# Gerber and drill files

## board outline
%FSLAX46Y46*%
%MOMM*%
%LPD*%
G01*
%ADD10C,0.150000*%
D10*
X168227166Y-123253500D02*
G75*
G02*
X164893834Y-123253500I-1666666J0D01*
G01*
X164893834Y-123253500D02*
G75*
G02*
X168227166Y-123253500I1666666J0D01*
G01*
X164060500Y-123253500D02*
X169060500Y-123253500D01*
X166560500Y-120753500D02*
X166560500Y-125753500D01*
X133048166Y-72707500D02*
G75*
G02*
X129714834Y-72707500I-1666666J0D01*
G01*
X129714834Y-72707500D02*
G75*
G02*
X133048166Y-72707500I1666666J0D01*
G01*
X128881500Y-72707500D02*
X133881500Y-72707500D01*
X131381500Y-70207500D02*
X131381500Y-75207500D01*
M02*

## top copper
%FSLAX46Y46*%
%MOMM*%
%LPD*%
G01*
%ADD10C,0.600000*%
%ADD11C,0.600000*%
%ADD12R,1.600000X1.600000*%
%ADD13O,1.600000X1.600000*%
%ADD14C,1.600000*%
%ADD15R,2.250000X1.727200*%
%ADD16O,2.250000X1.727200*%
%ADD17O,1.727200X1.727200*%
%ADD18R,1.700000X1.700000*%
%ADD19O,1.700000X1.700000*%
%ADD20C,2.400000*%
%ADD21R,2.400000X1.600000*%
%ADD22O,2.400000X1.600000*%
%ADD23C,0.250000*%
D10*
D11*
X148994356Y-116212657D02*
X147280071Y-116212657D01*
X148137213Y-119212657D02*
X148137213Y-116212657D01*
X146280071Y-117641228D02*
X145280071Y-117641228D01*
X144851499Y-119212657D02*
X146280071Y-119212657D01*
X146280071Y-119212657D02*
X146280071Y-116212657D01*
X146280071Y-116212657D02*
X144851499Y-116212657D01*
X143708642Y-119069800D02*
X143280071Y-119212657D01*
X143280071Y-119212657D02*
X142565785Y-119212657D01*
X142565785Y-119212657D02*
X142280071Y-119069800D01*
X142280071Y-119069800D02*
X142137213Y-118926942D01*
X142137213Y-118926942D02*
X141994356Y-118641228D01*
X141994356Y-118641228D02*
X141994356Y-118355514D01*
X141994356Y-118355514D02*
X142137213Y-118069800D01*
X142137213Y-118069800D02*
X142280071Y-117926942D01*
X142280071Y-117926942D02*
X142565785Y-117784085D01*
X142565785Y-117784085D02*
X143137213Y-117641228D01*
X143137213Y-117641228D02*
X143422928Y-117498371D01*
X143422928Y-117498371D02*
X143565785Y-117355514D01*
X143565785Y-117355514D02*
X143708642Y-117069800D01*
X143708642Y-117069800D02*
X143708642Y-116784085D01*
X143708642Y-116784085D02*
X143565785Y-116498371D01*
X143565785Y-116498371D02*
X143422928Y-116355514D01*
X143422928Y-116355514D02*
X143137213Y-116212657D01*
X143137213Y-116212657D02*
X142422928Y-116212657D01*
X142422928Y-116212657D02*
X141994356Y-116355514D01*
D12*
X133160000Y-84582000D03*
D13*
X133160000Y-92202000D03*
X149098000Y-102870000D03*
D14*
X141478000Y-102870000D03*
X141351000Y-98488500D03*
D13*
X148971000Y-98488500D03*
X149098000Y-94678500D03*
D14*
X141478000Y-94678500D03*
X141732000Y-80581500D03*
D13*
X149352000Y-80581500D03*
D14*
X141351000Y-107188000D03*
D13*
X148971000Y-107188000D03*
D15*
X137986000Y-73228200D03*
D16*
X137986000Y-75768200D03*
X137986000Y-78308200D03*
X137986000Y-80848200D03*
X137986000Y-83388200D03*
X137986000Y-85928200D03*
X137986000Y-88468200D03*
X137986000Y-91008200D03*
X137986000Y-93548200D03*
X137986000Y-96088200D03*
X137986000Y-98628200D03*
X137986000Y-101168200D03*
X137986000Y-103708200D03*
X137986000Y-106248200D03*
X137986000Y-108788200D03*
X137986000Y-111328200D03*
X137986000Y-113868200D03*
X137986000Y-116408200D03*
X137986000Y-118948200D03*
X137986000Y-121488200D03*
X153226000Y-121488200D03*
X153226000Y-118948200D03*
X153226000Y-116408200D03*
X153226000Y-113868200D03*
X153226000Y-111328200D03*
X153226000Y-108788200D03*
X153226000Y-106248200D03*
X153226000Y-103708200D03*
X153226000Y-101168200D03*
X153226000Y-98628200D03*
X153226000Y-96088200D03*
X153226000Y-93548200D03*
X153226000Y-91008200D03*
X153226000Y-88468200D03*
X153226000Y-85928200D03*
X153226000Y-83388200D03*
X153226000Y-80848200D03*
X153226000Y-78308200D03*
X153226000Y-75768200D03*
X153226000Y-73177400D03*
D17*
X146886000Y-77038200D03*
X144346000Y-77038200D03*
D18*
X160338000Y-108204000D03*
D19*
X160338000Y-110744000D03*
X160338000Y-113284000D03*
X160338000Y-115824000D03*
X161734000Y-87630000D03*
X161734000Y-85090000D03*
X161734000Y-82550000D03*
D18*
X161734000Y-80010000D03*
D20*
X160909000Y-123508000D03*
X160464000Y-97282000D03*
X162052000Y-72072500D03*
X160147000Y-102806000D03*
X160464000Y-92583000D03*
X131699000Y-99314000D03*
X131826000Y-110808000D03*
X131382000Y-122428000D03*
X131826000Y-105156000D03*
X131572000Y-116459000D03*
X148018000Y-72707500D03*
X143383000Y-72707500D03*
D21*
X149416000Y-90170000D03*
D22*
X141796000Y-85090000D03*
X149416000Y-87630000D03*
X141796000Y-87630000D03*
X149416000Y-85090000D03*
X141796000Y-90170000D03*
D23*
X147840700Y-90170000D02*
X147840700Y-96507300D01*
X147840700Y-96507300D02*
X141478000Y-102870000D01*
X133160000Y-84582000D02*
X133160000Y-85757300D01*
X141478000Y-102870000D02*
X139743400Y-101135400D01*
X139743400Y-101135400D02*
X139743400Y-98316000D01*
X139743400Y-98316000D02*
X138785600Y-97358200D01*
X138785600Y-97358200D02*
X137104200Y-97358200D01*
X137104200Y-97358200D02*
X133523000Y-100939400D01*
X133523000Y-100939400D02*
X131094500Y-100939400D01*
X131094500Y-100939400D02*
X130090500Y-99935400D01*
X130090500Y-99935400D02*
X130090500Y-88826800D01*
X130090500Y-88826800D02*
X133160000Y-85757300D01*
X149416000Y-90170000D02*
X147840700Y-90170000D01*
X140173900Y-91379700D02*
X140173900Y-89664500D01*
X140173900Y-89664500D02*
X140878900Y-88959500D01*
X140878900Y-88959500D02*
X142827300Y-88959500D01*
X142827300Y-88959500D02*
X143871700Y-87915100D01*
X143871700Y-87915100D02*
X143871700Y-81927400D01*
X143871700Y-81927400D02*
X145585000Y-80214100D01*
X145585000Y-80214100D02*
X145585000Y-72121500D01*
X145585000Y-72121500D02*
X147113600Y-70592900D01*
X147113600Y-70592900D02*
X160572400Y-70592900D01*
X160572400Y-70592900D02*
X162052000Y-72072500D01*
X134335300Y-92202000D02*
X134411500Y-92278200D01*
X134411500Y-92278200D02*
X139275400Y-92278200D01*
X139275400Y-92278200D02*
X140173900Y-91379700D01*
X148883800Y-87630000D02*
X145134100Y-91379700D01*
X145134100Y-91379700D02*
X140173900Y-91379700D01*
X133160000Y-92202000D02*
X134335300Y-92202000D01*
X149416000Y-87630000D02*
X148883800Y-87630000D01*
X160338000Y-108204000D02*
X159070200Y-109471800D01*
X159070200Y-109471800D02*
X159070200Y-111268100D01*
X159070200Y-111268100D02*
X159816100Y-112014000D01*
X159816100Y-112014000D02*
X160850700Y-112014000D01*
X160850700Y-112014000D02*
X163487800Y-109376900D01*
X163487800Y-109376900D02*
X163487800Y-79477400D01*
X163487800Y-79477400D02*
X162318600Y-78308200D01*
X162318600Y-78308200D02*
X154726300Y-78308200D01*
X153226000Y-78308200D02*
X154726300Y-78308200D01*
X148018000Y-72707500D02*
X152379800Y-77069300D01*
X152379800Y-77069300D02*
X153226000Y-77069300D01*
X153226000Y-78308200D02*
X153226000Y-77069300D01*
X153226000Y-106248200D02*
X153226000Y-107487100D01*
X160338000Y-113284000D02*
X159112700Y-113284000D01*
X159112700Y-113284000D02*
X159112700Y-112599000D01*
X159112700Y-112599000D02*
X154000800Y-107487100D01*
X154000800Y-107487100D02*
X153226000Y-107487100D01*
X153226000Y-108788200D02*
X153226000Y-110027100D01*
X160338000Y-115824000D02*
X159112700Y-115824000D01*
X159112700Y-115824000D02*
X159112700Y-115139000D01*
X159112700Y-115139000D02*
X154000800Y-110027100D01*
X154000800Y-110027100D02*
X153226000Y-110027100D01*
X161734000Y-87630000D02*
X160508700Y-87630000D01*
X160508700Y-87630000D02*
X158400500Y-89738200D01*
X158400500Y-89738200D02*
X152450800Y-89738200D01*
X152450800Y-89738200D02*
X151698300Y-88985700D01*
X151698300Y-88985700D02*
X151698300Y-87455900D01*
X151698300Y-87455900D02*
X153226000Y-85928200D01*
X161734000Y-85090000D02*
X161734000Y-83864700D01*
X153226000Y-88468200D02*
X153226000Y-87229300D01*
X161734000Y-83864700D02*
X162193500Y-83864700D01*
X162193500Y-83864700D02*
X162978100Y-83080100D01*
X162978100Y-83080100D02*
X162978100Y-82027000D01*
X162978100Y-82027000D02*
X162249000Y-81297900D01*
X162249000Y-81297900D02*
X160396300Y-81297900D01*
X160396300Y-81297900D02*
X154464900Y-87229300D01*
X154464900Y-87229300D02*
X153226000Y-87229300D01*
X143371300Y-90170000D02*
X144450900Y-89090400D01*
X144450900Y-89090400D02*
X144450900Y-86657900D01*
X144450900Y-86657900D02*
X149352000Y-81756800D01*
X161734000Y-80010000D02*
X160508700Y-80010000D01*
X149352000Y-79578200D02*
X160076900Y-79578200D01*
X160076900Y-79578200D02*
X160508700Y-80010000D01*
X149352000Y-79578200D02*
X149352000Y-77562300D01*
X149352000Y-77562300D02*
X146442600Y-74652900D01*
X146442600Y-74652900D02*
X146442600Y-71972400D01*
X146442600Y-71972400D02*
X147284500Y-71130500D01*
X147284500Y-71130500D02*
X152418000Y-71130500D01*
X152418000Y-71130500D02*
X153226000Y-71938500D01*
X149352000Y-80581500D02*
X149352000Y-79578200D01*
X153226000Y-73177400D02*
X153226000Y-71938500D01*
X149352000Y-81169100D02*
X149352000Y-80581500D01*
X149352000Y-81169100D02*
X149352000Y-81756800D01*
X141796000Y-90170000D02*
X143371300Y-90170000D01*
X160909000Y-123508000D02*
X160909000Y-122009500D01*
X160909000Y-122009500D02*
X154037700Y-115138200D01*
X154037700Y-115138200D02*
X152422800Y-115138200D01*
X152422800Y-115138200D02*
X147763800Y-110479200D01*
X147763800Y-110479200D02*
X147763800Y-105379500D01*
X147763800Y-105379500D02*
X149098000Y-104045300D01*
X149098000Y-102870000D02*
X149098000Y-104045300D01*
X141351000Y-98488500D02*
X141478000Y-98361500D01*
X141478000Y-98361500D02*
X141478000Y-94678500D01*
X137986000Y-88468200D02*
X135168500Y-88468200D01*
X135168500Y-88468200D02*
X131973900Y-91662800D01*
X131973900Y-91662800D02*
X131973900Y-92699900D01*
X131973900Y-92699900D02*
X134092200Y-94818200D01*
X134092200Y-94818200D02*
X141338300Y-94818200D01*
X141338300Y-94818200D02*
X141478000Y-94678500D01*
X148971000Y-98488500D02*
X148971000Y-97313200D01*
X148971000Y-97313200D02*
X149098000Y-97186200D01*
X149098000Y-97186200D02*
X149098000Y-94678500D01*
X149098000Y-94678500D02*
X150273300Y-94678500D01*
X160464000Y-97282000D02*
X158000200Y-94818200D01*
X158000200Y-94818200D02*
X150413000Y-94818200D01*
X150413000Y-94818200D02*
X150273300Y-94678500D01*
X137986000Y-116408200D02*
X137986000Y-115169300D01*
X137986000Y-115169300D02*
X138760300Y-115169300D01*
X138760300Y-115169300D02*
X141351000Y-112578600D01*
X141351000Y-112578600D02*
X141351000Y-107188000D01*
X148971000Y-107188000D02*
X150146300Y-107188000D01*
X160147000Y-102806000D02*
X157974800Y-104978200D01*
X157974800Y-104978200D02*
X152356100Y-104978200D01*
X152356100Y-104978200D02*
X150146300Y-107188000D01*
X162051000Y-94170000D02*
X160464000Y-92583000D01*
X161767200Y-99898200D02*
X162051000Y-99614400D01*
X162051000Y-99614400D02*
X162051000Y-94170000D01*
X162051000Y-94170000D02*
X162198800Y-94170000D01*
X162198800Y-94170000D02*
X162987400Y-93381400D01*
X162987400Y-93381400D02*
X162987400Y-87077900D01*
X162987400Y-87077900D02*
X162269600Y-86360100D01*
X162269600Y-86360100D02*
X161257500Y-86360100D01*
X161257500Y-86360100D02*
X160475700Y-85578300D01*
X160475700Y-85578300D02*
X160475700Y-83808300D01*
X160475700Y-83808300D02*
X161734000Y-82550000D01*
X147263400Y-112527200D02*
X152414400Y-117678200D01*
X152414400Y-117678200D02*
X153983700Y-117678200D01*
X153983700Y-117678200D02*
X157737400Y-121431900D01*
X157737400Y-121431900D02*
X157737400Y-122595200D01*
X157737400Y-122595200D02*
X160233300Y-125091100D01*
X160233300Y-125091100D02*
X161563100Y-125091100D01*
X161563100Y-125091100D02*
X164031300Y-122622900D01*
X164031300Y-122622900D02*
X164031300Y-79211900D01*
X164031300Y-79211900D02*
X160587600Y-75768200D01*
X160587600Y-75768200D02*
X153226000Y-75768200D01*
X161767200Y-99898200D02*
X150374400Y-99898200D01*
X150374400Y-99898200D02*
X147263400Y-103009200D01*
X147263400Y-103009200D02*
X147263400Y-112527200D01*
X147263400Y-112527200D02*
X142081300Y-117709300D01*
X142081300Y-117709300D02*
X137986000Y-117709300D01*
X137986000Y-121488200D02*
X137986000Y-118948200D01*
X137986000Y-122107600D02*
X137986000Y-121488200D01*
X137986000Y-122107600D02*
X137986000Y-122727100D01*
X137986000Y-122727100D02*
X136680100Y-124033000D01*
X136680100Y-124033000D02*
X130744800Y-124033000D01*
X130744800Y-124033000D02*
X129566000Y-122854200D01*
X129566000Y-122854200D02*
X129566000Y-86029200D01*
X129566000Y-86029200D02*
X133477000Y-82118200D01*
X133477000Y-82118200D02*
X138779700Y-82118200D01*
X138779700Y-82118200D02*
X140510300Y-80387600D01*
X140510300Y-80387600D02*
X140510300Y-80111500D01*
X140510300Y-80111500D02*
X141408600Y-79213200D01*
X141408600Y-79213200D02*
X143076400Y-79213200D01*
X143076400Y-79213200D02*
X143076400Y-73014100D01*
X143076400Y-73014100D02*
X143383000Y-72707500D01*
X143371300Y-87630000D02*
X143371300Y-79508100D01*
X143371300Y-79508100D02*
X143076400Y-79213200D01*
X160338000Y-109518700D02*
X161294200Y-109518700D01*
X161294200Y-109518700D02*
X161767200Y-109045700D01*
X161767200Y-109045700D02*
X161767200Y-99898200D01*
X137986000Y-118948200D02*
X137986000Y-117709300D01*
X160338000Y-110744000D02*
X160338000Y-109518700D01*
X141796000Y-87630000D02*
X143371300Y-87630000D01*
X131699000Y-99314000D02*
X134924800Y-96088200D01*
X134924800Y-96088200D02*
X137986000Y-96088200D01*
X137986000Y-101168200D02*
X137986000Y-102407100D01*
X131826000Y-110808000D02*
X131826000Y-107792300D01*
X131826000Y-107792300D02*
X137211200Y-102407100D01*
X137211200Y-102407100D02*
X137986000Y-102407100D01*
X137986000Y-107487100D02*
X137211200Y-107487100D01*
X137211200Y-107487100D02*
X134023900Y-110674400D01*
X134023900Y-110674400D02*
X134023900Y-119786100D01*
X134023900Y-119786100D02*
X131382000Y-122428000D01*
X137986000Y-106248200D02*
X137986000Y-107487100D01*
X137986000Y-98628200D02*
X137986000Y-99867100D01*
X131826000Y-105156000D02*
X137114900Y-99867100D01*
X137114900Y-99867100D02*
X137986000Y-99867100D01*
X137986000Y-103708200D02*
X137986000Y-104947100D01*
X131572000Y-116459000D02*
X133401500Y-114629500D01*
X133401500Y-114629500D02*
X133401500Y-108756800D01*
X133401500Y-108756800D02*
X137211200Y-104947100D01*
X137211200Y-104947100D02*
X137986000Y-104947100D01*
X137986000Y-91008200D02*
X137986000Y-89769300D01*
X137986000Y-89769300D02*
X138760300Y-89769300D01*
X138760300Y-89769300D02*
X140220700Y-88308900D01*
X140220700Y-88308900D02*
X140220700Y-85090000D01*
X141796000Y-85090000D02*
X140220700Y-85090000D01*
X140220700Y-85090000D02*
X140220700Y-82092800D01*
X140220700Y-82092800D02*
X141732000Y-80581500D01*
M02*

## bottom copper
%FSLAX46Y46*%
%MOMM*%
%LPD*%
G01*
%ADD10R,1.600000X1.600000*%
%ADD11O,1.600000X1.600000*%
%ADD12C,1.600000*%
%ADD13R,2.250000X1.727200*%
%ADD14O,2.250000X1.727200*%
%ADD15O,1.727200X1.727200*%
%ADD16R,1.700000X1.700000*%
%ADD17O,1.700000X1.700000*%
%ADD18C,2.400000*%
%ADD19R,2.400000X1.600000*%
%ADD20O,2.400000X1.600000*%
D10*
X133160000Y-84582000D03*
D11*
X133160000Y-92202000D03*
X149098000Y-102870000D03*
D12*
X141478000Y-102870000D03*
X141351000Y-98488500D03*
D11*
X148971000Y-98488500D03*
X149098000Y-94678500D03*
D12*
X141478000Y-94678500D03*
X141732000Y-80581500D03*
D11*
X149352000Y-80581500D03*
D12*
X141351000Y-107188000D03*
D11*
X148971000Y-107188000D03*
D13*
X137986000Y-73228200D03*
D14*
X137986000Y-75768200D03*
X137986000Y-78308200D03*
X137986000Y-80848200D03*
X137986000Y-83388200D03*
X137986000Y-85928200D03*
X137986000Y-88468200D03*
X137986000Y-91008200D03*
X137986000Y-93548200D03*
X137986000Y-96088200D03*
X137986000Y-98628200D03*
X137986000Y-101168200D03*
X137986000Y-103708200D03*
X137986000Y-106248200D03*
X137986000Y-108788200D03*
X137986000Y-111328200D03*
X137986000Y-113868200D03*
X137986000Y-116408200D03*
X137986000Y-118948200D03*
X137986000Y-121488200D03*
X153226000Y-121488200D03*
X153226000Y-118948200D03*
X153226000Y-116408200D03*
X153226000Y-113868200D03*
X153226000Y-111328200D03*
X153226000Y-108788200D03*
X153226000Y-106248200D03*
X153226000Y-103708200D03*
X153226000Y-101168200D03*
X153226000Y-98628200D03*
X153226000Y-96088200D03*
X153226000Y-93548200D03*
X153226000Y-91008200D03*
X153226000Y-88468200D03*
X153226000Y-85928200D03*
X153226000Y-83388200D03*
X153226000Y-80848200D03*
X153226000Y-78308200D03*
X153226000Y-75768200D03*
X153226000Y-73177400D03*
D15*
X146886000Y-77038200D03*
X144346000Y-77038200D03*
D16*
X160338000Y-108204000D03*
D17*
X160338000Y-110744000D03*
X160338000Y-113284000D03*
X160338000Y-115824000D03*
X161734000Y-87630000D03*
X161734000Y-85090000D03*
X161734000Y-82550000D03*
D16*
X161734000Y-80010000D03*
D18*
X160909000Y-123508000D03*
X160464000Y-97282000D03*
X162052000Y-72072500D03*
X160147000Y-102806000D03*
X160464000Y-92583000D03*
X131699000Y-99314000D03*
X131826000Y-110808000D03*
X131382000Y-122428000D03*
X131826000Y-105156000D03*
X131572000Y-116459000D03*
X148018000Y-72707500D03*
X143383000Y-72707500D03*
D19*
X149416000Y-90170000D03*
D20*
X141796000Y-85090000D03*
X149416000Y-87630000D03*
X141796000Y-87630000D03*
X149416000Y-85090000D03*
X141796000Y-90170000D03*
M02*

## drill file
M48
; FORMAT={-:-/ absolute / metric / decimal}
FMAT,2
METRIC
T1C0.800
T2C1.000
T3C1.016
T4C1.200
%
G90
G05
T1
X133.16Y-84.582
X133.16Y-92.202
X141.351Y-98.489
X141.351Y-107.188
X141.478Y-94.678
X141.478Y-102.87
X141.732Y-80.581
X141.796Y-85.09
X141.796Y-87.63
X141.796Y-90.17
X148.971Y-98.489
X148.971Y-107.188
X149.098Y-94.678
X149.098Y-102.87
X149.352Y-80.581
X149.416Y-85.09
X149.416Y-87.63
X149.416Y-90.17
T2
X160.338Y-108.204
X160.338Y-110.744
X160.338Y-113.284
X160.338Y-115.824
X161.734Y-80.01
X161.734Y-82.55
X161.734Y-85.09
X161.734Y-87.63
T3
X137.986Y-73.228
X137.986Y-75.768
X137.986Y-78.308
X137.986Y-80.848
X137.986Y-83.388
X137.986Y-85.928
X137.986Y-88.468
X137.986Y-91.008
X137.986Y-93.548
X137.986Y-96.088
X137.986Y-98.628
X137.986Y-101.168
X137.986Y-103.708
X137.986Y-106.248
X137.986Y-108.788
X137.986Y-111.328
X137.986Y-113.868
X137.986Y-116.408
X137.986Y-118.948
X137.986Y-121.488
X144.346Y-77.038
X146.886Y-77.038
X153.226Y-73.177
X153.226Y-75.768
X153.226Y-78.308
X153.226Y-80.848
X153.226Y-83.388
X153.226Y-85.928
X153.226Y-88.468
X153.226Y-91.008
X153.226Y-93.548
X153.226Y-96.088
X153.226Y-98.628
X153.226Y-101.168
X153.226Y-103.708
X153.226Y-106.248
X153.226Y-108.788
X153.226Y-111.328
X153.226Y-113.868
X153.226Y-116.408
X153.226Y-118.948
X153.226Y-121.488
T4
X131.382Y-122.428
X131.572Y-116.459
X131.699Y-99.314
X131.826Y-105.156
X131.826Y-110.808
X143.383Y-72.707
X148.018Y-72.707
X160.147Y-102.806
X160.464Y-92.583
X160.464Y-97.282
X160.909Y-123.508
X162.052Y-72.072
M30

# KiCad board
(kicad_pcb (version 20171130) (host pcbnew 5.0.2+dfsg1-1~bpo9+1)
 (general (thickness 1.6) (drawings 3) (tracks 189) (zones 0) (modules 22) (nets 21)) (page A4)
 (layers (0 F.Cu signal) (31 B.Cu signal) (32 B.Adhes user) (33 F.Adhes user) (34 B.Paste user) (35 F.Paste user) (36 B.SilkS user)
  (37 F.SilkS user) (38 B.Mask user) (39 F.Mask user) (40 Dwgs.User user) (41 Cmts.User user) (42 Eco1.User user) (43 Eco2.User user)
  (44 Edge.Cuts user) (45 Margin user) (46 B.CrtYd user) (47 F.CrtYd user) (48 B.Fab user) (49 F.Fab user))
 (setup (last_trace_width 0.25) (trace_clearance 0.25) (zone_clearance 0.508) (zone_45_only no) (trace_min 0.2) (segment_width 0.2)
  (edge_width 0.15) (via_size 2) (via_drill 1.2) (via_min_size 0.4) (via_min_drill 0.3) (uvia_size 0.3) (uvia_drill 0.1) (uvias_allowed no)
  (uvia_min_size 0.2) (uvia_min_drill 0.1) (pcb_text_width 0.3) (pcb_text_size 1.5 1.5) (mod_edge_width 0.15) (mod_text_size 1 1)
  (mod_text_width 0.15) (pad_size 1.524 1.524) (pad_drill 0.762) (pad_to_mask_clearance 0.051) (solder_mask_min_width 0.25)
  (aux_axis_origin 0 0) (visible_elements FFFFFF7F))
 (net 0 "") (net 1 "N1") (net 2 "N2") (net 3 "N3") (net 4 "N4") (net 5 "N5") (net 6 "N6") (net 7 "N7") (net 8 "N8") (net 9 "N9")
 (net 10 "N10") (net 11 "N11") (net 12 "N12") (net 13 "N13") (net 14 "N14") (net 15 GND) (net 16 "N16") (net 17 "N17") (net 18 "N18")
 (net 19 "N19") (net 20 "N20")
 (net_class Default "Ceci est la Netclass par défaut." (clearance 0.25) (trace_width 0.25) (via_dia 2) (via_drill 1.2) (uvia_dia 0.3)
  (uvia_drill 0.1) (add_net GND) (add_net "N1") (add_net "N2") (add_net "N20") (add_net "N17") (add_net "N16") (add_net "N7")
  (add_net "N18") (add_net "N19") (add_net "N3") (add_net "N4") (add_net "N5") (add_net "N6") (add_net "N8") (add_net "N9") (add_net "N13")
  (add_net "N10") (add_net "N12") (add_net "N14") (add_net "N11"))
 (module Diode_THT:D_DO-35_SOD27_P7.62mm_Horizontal (layer F.Cu) (at 133.16 84.582 270)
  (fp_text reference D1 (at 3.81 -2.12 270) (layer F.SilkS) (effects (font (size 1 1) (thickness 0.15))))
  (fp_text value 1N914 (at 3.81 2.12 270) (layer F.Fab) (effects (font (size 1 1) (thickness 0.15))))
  (pad 1 thru_hole rect (at 0 0 270) (size 1.6 1.6) (drill 0.8) (layers *.Cu *.Mask) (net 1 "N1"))
  (pad 2 thru_hole oval (at 7.62 0 270) (size 1.6 1.6) (drill 0.8) (layers *.Cu *.Mask) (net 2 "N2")))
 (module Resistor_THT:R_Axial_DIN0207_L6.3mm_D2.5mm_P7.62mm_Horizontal (layer F.Cu) (at 141.478 102.87)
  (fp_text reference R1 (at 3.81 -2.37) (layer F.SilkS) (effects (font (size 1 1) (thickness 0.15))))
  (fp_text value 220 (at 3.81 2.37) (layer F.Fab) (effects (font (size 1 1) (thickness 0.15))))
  (pad 2 thru_hole oval (at 7.62 0) (size 1.6 1.6) (drill 0.8) (layers *.Cu *.Mask) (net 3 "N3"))
  (pad 1 thru_hole circle (at 0 0) (size 1.6 1.6) (drill 0.8) (layers *.Cu *.Mask) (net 1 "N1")))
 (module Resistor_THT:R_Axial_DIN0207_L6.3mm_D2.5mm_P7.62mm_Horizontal (layer F.Cu) (at 141.351 98.4885)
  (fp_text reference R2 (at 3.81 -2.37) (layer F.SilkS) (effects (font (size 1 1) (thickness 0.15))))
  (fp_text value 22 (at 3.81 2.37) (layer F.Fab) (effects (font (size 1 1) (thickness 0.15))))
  (pad 1 thru_hole circle (at 0 0) (size 1.6 1.6) (drill 0.8) (layers *.Cu *.Mask) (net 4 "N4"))
  (pad 2 thru_hole oval (at 7.62 0) (size 1.6 1.6) (drill 0.8) (layers *.Cu *.Mask) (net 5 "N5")))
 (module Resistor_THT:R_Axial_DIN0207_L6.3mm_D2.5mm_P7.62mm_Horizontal (layer F.Cu) (at 141.478 94.6785)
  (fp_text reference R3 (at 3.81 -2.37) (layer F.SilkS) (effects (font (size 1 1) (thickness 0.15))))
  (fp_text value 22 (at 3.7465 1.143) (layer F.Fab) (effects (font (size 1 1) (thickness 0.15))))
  (pad 2 thru_hole oval (at 7.62 0) (size 1.6 1.6) (drill 0.8) (layers *.Cu *.Mask) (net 5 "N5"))
  (pad 1 thru_hole circle (at 0 0) (size 1.6 1.6) (drill 0.8) (layers *.Cu *.Mask) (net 4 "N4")))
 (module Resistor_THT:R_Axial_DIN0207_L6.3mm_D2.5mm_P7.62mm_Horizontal (layer F.Cu) (at 141.732 80.5815)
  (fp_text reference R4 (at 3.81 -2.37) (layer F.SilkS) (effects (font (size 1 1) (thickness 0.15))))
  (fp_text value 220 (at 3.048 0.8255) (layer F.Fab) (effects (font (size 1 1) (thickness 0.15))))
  (pad 1 thru_hole circle (at 0 0) (size 1.6 1.6) (drill 0.8) (layers *.Cu *.Mask) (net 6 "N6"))
  (pad 2 thru_hole oval (at 7.62 0) (size 1.6 1.6) (drill 0.8) (layers *.Cu *.Mask) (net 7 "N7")))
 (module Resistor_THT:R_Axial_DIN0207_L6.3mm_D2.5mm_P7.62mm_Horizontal (layer F.Cu) (at 141.351 107.188)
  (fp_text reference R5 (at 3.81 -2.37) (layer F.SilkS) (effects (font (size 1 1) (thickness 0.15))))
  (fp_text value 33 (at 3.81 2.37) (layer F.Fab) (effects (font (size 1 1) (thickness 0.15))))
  (pad 1 thru_hole circle (at 0 0) (size 1.6 1.6) (drill 0.8) (layers *.Cu *.Mask) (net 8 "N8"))
  (pad 2 thru_hole oval (at 7.62 0) (size 1.6 1.6) (drill 0.8) (layers *.Cu *.Mask) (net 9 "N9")))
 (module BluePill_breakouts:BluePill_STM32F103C (layer F.Cu) (at 137.986 73.279)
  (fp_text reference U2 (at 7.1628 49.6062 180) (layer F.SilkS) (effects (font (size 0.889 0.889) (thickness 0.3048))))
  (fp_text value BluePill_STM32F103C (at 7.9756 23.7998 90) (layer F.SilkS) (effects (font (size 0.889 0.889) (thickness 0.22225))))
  (pad 1 thru_hole rect (at 0 -0.0508 270) (size 1.7272 2.25) (drill 1.016) (layers *.Cu *.Mask F.SilkS))
  (pad 2 thru_hole oval (at 0 2.4892 270) (size 1.7272 2.25) (drill 1.016) (layers *.Cu *.Mask F.SilkS))
  (pad 3 thru_hole oval (at 0 5.0292 270) (size 1.7272 2.25) (drill 1.016) (layers *.Cu *.Mask F.SilkS))
  (pad 4 thru_hole oval (at 0 7.5692 270) (size 1.7272 2.25) (drill 1.016) (layers *.Cu *.Mask F.SilkS))
  (pad 5 thru_hole oval (at 0 10.1092 270) (size 1.7272 2.25) (drill 1.016) (layers *.Cu *.Mask F.SilkS))
  (pad 6 thru_hole oval (at 0 12.6492 270) (size 1.7272 2.25) (drill 1.016) (layers *.Cu *.Mask F.SilkS))
  (pad 7 thru_hole oval (at 0 15.1892 270) (size 1.7272 2.25) (drill 1.016) (layers *.Cu *.Mask F.SilkS) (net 4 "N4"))
  (pad 8 thru_hole oval (at 0 17.7292 270) (size 1.7272 2.25) (drill 1.016) (layers *.Cu *.Mask F.SilkS) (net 6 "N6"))
  (pad 9 thru_hole oval (at 0 20.2692 270) (size 1.7272 2.25) (drill 1.016) (layers *.Cu *.Mask F.SilkS))
  (pad 10 thru_hole oval (at 0 22.8092 270) (size 1.7272 2.25) (drill 1.016) (layers *.Cu *.Mask F.SilkS) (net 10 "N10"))
  (pad 11 thru_hole oval (at 0 25.3492 270) (size 1.7272 2.25) (drill 1.016) (layers *.Cu *.Mask F.SilkS) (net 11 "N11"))
  (pad 12 thru_hole oval (at 0 27.8892 270) (size 1.7272 2.25) (drill 1.016) (layers *.Cu *.Mask F.SilkS) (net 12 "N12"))
  (pad 13 thru_hole oval (at 0 30.4292 270) (size 1.7272 2.25) (drill 1.016) (layers *.Cu *.Mask F.SilkS) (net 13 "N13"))
  (pad 14 thru_hole oval (at 0 32.9692 270) (size 1.7272 2.25) (drill 1.016) (layers *.Cu *.Mask F.SilkS) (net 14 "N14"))
  (pad 15 thru_hole oval (at 0 35.5092 270) (size 1.7272 2.25) (drill 1.016) (layers *.Cu *.Mask F.SilkS))
  (pad 16 thru_hole oval (at 0 38.0492 270) (size 1.7272 2.25) (drill 1.016) (layers *.Cu *.Mask F.SilkS))
  (pad 17 thru_hole oval (at 0 40.5892 270) (size 1.7272 2.25) (drill 1.016) (layers *.Cu *.Mask F.SilkS))
  (pad 18 thru_hole oval (at 0 43.1292 270) (size 1.7272 2.25) (drill 1.016) (layers *.Cu *.Mask F.SilkS) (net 8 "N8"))
  (pad 19 thru_hole oval (at 0 45.6692 270) (size 1.7272 2.25) (drill 1.016) (layers *.Cu *.Mask F.SilkS) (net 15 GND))
  (pad 20 thru_hole oval (at 0 48.2092 270) (size 1.7272 2.25) (drill 1.016) (layers *.Cu *.Mask F.SilkS) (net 15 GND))
  (pad 21 thru_hole oval (at 15.24 48.2092 90) (size 1.7272 2.25) (drill 1.016) (layers *.Cu *.Mask F.SilkS))
  (pad 22 thru_hole oval (at 15.24 45.6692 90) (size 1.7272 2.25) (drill 1.016) (layers *.Cu *.Mask F.SilkS))
  (pad 23 thru_hole oval (at 15.24 43.1292 90) (size 1.7272 2.25) (drill 1.016) (layers *.Cu *.Mask F.SilkS))
  (pad 24 thru_hole oval (at 15.24 40.5892 90) (size 1.7272 2.25) (drill 1.016) (layers *.Cu *.Mask F.SilkS))
  (pad 25 thru_hole oval (at 15.24 38.0492 90) (size 1.7272 2.25) (drill 1.016) (layers *.Cu *.Mask F.SilkS))
  (pad 26 thru_hole oval (at 15.24 35.5092 90) (size 1.7272 2.25) (drill 1.016) (layers *.Cu *.Mask F.SilkS) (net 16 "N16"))
  (pad 27 thru_hole oval (at 15.24 32.9692 90) (size 1.7272 2.25) (drill 1.016) (layers *.Cu *.Mask F.SilkS) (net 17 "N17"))
  (pad 28 thru_hole oval (at 15.24 30.4292 90) (size 1.7272 2.25) (drill 1.016) (layers *.Cu *.Mask F.SilkS))
  (pad 29 thru_hole oval (at 15.24 27.8892 90) (size 1.7272 2.25) (drill 1.016) (layers *.Cu *.Mask F.SilkS))
  (pad 30 thru_hole oval (at 15.24 25.3492 90) (size 1.7272 2.25) (drill 1.016) (layers *.Cu *.Mask F.SilkS))
  (pad 31 thru_hole oval (at 15.24 22.8092 90) (size 1.7272 2.25) (drill 1.016) (layers *.Cu *.Mask F.SilkS))
  (pad 32 thru_hole oval (at 15.24 20.2692 90) (size 1.7272 2.25) (drill 1.016) (layers *.Cu *.Mask F.SilkS))
  (pad 33 thru_hole oval (at 15.24 17.7292 90) (size 1.7272 2.25) (drill 1.016) (layers *.Cu *.Mask F.SilkS))
  (pad 34 thru_hole oval (at 15.24 15.1892 90) (size 1.7272 2.25) (drill 1.016) (layers *.Cu *.Mask F.SilkS) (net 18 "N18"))
  (pad 35 thru_hole oval (at 15.24 12.6492 90) (size 1.7272 2.25) (drill 1.016) (layers *.Cu *.Mask F.SilkS) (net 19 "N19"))
  (pad 36 thru_hole oval (at 15.24 10.1092 90) (size 1.7272 2.25) (drill 1.016) (layers *.Cu *.Mask F.SilkS))
  (pad 37 thru_hole oval (at 15.24 7.5692 90) (size 1.7272 2.25) (drill 1.016) (layers *.Cu *.Mask F.SilkS))
  (pad 38 thru_hole oval (at 15.24 5.0292 90) (size 1.7272 2.25) (drill 1.016) (layers *.Cu *.Mask F.SilkS) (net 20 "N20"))
  (pad 39 thru_hole oval (at 15.24 2.4892 90) (size 1.7272 2.25) (drill 1.016) (layers *.Cu *.Mask F.SilkS) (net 15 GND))
  (pad 40 thru_hole oval (at 15.24 -0.1016 90) (size 1.7272 2.25) (drill 1.016) (layers *.Cu *.Mask F.SilkS) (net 7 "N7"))
  (pad 41 thru_hole oval (at 8.9 3.7592 90) (size 1.7272 1.7272) (drill 1.016) (layers *.Cu *.Mask F.SilkS))
  (pad 42 thru_hole oval (at 6.36 3.7592 90) (size 1.7272 1.7272) (drill 1.016) (layers *.Cu *.Mask F.SilkS)))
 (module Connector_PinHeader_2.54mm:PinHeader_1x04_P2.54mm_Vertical (layer F.Cu) (at 160.338 108.204)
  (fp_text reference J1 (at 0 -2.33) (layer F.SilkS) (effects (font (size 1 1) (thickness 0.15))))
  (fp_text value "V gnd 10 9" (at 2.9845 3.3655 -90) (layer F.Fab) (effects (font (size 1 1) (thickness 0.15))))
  (pad 1 thru_hole rect (at 0 0) (size 1.7 1.7) (drill 1) (layers *.Cu *.Mask) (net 20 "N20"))
  (pad 2 thru_hole oval (at 0 2.54) (size 1.7 1.7) (drill 1) (layers *.Cu *.Mask) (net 15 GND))
  (pad 3 thru_hole oval (at 0 5.08) (size 1.7 1.7) (drill 1) (layers *.Cu *.Mask) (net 17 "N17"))
  (pad 4 thru_hole oval (at 0 7.62) (size 1.7 1.7) (drill 1) (layers *.Cu *.Mask) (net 16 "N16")))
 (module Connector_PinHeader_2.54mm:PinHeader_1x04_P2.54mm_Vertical (layer F.Cu) (at 161.734 80.01)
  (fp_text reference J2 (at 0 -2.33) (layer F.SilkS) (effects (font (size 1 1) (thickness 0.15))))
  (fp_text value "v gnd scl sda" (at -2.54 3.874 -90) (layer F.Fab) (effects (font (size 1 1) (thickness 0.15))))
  (pad 4 thru_hole oval (at 0 7.62) (size 1.7 1.7) (drill 1) (layers *.Cu *.Mask) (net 19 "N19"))
  (pad 3 thru_hole oval (at 0 5.08) (size 1.7 1.7) (drill 1) (layers *.Cu *.Mask) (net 18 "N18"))
  (pad 2 thru_hole oval (at 0 2.54) (size 1.7 1.7) (drill 1) (layers *.Cu *.Mask) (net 15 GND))
  (pad 1 thru_hole rect (at 0 0) (size 1.7 1.7) (drill 1) (layers *.Cu *.Mask) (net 7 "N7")))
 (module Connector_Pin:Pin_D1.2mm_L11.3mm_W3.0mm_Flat (layer F.Cu) (at 160.909 123.508)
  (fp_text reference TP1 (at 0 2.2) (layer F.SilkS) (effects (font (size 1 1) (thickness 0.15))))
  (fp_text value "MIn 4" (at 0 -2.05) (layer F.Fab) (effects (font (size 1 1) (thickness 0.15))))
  (pad 1 thru_hole circle (at 0 0) (size 2.4 2.4) (drill 1.2) (layers *.Cu *.Mask) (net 3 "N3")))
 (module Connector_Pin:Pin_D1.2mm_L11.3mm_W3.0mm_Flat (layer F.Cu) (at 160.464 97.282)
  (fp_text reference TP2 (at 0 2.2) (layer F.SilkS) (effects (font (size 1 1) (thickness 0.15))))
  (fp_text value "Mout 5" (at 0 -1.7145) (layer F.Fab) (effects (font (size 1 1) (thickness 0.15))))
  (pad 1 thru_hole circle (at 0 0) (size 2.4 2.4) (drill 1.2) (layers *.Cu *.Mask) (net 5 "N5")))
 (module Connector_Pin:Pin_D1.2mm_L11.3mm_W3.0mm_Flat (layer F.Cu) (at 162.052 72.0725)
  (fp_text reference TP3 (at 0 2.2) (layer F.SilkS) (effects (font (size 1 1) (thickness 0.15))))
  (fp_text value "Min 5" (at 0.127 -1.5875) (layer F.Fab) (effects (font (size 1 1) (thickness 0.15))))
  (pad 1 thru_hole circle (at 0 0) (size 2.4 2.4) (drill 1.2) (layers *.Cu *.Mask) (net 2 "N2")))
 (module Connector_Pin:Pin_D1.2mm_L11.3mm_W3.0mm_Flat (layer F.Cu) (at 160.147 102.806)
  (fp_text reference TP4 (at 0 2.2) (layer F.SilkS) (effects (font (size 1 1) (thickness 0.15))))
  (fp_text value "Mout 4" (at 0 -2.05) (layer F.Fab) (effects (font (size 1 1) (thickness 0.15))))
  (pad 1 thru_hole circle (at 0 0) (size 2.4 2.4) (drill 1.2) (layers *.Cu *.Mask) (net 9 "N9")))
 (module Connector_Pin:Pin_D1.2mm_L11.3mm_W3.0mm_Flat (layer F.Cu) (at 160.464 92.583)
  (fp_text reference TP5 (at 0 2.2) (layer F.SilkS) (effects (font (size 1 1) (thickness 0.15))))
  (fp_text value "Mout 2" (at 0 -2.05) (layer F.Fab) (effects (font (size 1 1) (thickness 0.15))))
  (pad 1 thru_hole circle (at 0 0) (size 2.4 2.4) (drill 1.2) (layers *.Cu *.Mask) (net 15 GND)))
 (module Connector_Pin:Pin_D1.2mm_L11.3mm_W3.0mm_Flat (layer F.Cu) (at 131.699 99.314)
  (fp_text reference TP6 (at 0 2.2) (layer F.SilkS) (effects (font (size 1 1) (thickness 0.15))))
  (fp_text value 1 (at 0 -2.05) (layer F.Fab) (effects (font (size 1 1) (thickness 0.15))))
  (pad 1 thru_hole circle (at 0 0) (size 2.4 2.4) (drill 1.2) (layers *.Cu *.Mask) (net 10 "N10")))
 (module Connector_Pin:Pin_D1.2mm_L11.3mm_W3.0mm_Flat (layer F.Cu) (at 131.826 110.808)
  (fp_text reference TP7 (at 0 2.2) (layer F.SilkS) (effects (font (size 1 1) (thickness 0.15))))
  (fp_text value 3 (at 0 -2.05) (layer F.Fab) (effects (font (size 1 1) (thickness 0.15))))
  (pad 1 thru_hole circle (at 0 0) (size 2.4 2.4) (drill 1.2) (layers *.Cu *.Mask) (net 12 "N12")))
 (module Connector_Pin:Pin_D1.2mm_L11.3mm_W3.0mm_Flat (layer F.Cu) (at 131.382 122.428)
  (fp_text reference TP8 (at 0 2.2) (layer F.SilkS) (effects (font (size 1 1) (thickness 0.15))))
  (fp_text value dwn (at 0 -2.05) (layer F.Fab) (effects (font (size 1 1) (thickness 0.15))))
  (pad 1 thru_hole circle (at 0 0) (size 2.4 2.4) (drill 1.2) (layers *.Cu *.Mask) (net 14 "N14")))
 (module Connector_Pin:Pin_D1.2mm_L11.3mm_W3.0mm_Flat (layer F.Cu) (at 131.826 105.156)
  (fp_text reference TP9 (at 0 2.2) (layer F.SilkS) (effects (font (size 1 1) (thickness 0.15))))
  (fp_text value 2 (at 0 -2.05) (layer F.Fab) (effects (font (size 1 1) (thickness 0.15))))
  (pad 1 thru_hole circle (at 0 0) (size 2.4 2.4) (drill 1.2) (layers *.Cu *.Mask) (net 11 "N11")))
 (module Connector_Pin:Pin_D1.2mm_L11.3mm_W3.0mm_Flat (layer F.Cu) (at 131.572 116.459)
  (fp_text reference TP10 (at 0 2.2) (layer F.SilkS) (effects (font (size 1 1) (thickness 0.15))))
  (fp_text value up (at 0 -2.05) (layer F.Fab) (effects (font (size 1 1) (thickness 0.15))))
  (pad 1 thru_hole circle (at 0 0) (size 2.4 2.4) (drill 1.2) (layers *.Cu *.Mask) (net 13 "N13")))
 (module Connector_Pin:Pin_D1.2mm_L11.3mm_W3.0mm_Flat (layer F.Cu) (at 148.018 72.7075)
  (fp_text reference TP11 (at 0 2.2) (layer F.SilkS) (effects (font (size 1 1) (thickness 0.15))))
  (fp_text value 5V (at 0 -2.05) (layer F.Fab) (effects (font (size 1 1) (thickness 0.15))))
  (pad 1 thru_hole circle (at 0 0) (size 2.4 2.4) (drill 1.2) (layers *.Cu *.Mask) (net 20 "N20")))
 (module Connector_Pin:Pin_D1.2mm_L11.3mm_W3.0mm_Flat (layer F.Cu) (at 143.383 72.7075)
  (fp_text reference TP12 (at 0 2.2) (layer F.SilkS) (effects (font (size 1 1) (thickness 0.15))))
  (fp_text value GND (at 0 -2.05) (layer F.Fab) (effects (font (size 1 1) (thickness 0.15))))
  (pad 1 thru_hole circle (at 0 0) (size 2.4 2.4) (drill 1.2) (layers *.Cu *.Mask) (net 15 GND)))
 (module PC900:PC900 (layer F.Cu) (at 149.416 90.17 180)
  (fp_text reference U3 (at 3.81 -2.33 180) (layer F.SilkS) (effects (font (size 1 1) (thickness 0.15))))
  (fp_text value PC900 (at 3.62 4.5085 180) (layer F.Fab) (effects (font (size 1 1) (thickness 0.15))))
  (pad 1 thru_hole rect (at 0 0 180) (size 2.4 1.6) (drill 0.8) (layers *.Cu *.Mask) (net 1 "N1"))
  (pad 4 thru_hole oval (at 7.62 5.08 180) (size 2.4 1.6) (drill 0.8) (layers *.Cu *.Mask) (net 6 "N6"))
  (pad 2 thru_hole oval (at 0 2.54 180) (size 2.4 1.6) (drill 0.8) (layers *.Cu *.Mask) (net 2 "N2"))
  (pad 5 thru_hole oval (at 7.62 2.54 180) (size 2.4 1.6) (drill 0.8) (layers *.Cu *.Mask) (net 15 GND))
  (pad 3 thru_hole oval (at 0 5.08 180) (size 2.4 1.6) (drill 0.8) (layers *.Cu *.Mask))
  (pad 6 thru_hole oval (at 7.62 0 180) (size 2.4 1.6) (drill 0.8) (layers *.Cu *.Mask) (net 7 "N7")))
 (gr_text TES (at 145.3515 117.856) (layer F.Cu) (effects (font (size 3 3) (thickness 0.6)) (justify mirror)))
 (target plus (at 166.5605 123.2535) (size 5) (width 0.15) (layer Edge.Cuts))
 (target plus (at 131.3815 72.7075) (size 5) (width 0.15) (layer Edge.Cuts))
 (segment (start 147.8407 90.17) (end 147.8407 96.5073) (width 0.25) (layer F.Cu) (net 1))
 (segment (start 147.8407 96.5073) (end 141.478 102.87) (width 0.25) (layer F.Cu) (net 1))
 (segment (start 133.16 84.582) (end 133.16 85.7573) (width 0.25) (layer F.Cu) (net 1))
 (segment (start 141.478 102.87) (end 139.7434 101.1354) (width 0.25) (layer F.Cu) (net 1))
 (segment (start 139.7434 101.1354) (end 139.7434 98.316) (width 0.25) (layer F.Cu) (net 1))
 (segment (start 139.7434 98.316) (end 138.7856 97.3582) (width 0.25) (layer F.Cu) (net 1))
 (segment (start 138.7856 97.3582) (end 137.1042 97.3582) (width 0.25) (layer F.Cu) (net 1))
 (segment (start 137.1042 97.3582) (end 133.523 100.9394) (width 0.25) (layer F.Cu) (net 1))
 (segment (start 133.523 100.9394) (end 131.0945 100.9394) (width 0.25) (layer F.Cu) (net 1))
 (segment (start 131.0945 100.9394) (end 130.0905 99.9354) (width 0.25) (layer F.Cu) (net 1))
 (segment (start 130.0905 99.9354) (end 130.0905 88.8268) (width 0.25) (layer F.Cu) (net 1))
 (segment (start 130.0905 88.8268) (end 133.16 85.7573) (width 0.25) (layer F.Cu) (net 1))
 (segment (start 149.416 90.17) (end 147.8407 90.17) (width 0.25) (layer F.Cu) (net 1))
 (segment (start 140.1739 91.3797) (end 140.1739 89.6645) (width 0.25) (layer F.Cu) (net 2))
 (segment (start 140.1739 89.6645) (end 140.8789 88.9595) (width 0.25) (layer F.Cu) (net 2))
 (segment (start 140.8789 88.9595) (end 142.8273 88.9595) (width 0.25) (layer F.Cu) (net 2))
 (segment (start 142.8273 88.9595) (end 143.8717 87.9151) (width 0.25) (layer F.Cu) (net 2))
 (segment (start 143.8717 87.9151) (end 143.8717 81.9274) (width 0.25) (layer F.Cu) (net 2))
 (segment (start 143.8717 81.9274) (end 145.585 80.2141) (width 0.25) (layer F.Cu) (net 2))
 (segment (start 145.585 80.2141) (end 145.585 72.1215) (width 0.25) (layer F.Cu) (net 2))
 (segment (start 145.585 72.1215) (end 147.1136 70.5929) (width 0.25) (layer F.Cu) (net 2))
 (segment (start 147.1136 70.5929) (end 160.5724 70.5929) (width 0.25) (layer F.Cu) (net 2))
 (segment (start 160.5724 70.5929) (end 162.052 72.0725) (width 0.25) (layer F.Cu) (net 2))
 (segment (start 134.3353 92.202) (end 134.4115 92.2782) (width 0.25) (layer F.Cu) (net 2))
 (segment (start 134.4115 92.2782) (end 139.2754 92.2782) (width 0.25) (layer F.Cu) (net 2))
 (segment (start 139.2754 92.2782) (end 140.1739 91.3797) (width 0.25) (layer F.Cu) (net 2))
 (segment (start 148.8838 87.63) (end 145.1341 91.3797) (width 0.25) (layer F.Cu) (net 2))
 (segment (start 145.1341 91.3797) (end 140.1739 91.3797) (width 0.25) (layer F.Cu) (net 2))
 (segment (start 133.16 92.202) (end 134.3353 92.202) (width 0.25) (layer F.Cu) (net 2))
 (segment (start 149.416 87.63) (end 148.8838 87.63) (width 0.25) (layer F.Cu) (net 2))
 (segment (start 160.338 108.204) (end 159.0702 109.4718) (width 0.25) (layer F.Cu) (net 20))
 (segment (start 159.0702 109.4718) (end 159.0702 111.2681) (width 0.25) (layer F.Cu) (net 20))
 (segment (start 159.0702 111.2681) (end 159.8161 112.014) (width 0.25) (layer F.Cu) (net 20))
 (segment (start 159.8161 112.014) (end 160.8507 112.014) (width 0.25) (layer F.Cu) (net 20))
 (segment (start 160.8507 112.014) (end 163.4878 109.3769) (width 0.25) (layer F.Cu) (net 20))
 (segment (start 163.4878 109.3769) (end 163.4878 79.4774) (width 0.25) (layer F.Cu) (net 20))
 (segment (start 163.4878 79.4774) (end 162.3186 78.3082) (width 0.25) (layer F.Cu) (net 20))
 (segment (start 162.3186 78.3082) (end 154.7263 78.3082) (width 0.25) (layer F.Cu) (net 20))
 (segment (start 153.226 78.3082) (end 154.7263 78.3082) (width 0.25) (layer F.Cu) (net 20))
 (segment (start 148.018 72.7075) (end 152.3798 77.0693) (width 0.25) (layer F.Cu) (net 20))
 (segment (start 152.3798 77.0693) (end 153.226 77.0693) (width 0.25) (layer F.Cu) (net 20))
 (segment (start 153.226 78.3082) (end 153.226 77.0693) (width 0.25) (layer F.Cu) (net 20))
 (segment (start 153.226 106.2482) (end 153.226 107.4871) (width 0.25) (layer F.Cu) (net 17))
 (segment (start 160.338 113.284) (end 159.1127 113.284) (width 0.25) (layer F.Cu) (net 17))
 (segment (start 159.1127 113.284) (end 159.1127 112.599) (width 0.25) (layer F.Cu) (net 17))
 (segment (start 159.1127 112.599) (end 154.0008 107.4871) (width 0.25) (layer F.Cu) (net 17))
 (segment (start 154.0008 107.4871) (end 153.226 107.4871) (width 0.25) (layer F.Cu) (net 17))
 (segment (start 153.226 108.7882) (end 153.226 110.0271) (width 0.25) (layer F.Cu) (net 16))
 (segment (start 160.338 115.824) (end 159.1127 115.824) (width 0.25) (layer F.Cu) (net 16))
 (segment (start 159.1127 115.824) (end 159.1127 115.139) (width 0.25) (layer F.Cu) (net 16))
 (segment (start 159.1127 115.139) (end 154.0008 110.0271) (width 0.25) (layer F.Cu) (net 16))
 (segment (start 154.0008 110.0271) (end 153.226 110.0271) (width 0.25) (layer F.Cu) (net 16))
 (segment (start 161.734 87.63) (end 160.5087 87.63) (width 0.25) (layer F.Cu) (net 19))
 (segment (start 160.5087 87.63) (end 158.4005 89.7382) (width 0.25) (layer F.Cu) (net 19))
 (segment (start 158.4005 89.7382) (end 152.4508 89.7382) (width 0.25) (layer F.Cu) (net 19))
 (segment (start 152.4508 89.7382) (end 151.6983 88.9857) (width 0.25) (layer F.Cu) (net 19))
 (segment (start 151.6983 88.9857) (end 151.6983 87.4559) (width 0.25) (layer F.Cu) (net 19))
 (segment (start 151.6983 87.4559) (end 153.226 85.9282) (width 0.25) (layer F.Cu) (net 19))
 (segment (start 161.734 85.09) (end 161.734 83.8647) (width 0.25) (layer F.Cu) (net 18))
 (segment (start 153.226 88.4682) (end 153.226 87.2293) (width 0.25) (layer F.Cu) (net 18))
 (segment (start 161.734 83.8647) (end 162.1935 83.8647) (width 0.25) (layer F.Cu) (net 18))
 (segment (start 162.1935 83.8647) (end 162.9781 83.0801) (width 0.25) (layer F.Cu) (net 18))
 (segment (start 162.9781 83.0801) (end 162.9781 82.027) (width 0.25) (layer F.Cu) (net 18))
 (segment (start 162.9781 82.027) (end 162.249 81.2979) (width 0.25) (layer F.Cu) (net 18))
 (segment (start 162.249 81.2979) (end 160.3963 81.2979) (width 0.25) (layer F.Cu) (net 18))
 (segment (start 160.3963 81.2979) (end 154.4649 87.2293) (width 0.25) (layer F.Cu) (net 18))
 (segment (start 154.4649 87.2293) (end 153.226 87.2293) (width 0.25) (layer F.Cu) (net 18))
 (segment (start 143.3713 90.17) (end 144.4509 89.0904) (width 0.25) (layer F.Cu) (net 7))
 (segment (start 144.4509 89.0904) (end 144.4509 86.6579) (width 0.25) (layer F.Cu) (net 7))
 (segment (start 144.4509 86.6579) (end 149.352 81.7568) (width 0.25) (layer F.Cu) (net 7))
 (segment (start 161.734 80.01) (end 160.5087 80.01) (width 0.25) (layer F.Cu) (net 7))
 (segment (start 149.352 79.5782) (end 160.0769 79.5782) (width 0.25) (layer F.Cu) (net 7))
 (segment (start 160.0769 79.5782) (end 160.5087 80.01) (width 0.25) (layer F.Cu) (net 7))
 (segment (start 149.352 79.5782) (end 149.352 77.5623) (width 0.25) (layer F.Cu) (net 7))
 (segment (start 149.352 77.5623) (end 146.4426 74.6529) (width 0.25) (layer F.Cu) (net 7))
 (segment (start 146.4426 74.6529) (end 146.4426 71.9724) (width 0.25) (layer F.Cu) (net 7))
 (segment (start 146.4426 71.9724) (end 147.2845 71.1305) (width 0.25) (layer F.Cu) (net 7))
 (segment (start 147.2845 71.1305) (end 152.418 71.1305) (width 0.25) (layer F.Cu) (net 7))
 (segment (start 152.418 71.1305) (end 153.226 71.9385) (width 0.25) (layer F.Cu) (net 7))
 (segment (start 149.352 80.5815) (end 149.352 79.5782) (width 0.25) (layer F.Cu) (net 7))
 (segment (start 153.226 73.1774) (end 153.226 71.9385) (width 0.25) (layer F.Cu) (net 7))
 (segment (start 149.352 81.1691) (end 149.352 80.5815) (width 0.25) (layer F.Cu) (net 7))
 (segment (start 149.352 81.1691) (end 149.352 81.7568) (width 0.25) (layer F.Cu) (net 7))
 (segment (start 141.796 90.17) (end 143.3713 90.17) (width 0.25) (layer F.Cu) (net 7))
 (segment (start 160.909 123.508) (end 160.909 122.0095) (width 0.25) (layer F.Cu) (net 3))
 (segment (start 160.909 122.0095) (end 154.0377 115.1382) (width 0.25) (layer F.Cu) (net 3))
 (segment (start 154.0377 115.1382) (end 152.4228 115.1382) (width 0.25) (layer F.Cu) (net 3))
 (segment (start 152.4228 115.1382) (end 147.7638 110.4792) (width 0.25) (layer F.Cu) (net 3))
 (segment (start 147.7638 110.4792) (end 147.7638 105.3795) (width 0.25) (layer F.Cu) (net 3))
 (segment (start 147.7638 105.3795) (end 149.098 104.0453) (width 0.25) (layer F.Cu) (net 3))
 (segment (start 149.098 102.87) (end 149.098 104.0453) (width 0.25) (layer F.Cu) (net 3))
 (segment (start 141.351 98.4885) (end 141.478 98.3615) (width 0.25) (layer F.Cu) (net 4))
 (segment (start 141.478 98.3615) (end 141.478 94.6785) (width 0.25) (layer F.Cu) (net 4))
 (segment (start 137.986 88.4682) (end 135.1685 88.4682) (width 0.25) (layer F.Cu) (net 4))
 (segment (start 135.1685 88.4682) (end 131.9739 91.6628) (width 0.25) (layer F.Cu) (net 4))
 (segment (start 131.9739 91.6628) (end 131.9739 92.6999) (width 0.25) (layer F.Cu) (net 4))
 (segment (start 131.9739 92.6999) (end 134.0922 94.8182) (width 0.25) (layer F.Cu) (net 4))
 (segment (start 134.0922 94.8182) (end 141.3383 94.8182) (width 0.25) (layer F.Cu) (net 4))
 (segment (start 141.3383 94.8182) (end 141.478 94.6785) (width 0.25) (layer F.Cu) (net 4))
 (segment (start 148.971 98.4885) (end 148.971 97.3132) (width 0.25) (layer F.Cu) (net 5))
 (segment (start 148.971 97.3132) (end 149.098 97.1862) (width 0.25) (layer F.Cu) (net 5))
 (segment (start 149.098 97.1862) (end 149.098 94.6785) (width 0.25) (layer F.Cu) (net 5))
 (segment (start 149.098 94.6785) (end 150.2733 94.6785) (width 0.25) (layer F.Cu) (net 5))
 (segment (start 160.464 97.282) (end 158.0002 94.8182) (width 0.25) (layer F.Cu) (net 5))
 (segment (start 158.0002 94.8182) (end 150.413 94.8182) (width 0.25) (layer F.Cu) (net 5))
 (segment (start 150.413 94.8182) (end 150.2733 94.6785) (width 0.25) (layer F.Cu) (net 5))
 (segment (start 137.986 116.4082) (end 137.986 115.1693) (width 0.25) (layer F.Cu) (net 8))
 (segment (start 137.986 115.1693) (end 138.7603 115.1693) (width 0.25) (layer F.Cu) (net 8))
 (segment (start 138.7603 115.1693) (end 141.351 112.5786) (width 0.25) (layer F.Cu) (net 8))
 (segment (start 141.351 112.5786) (end 141.351 107.188) (width 0.25) (layer F.Cu) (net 8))
 (segment (start 148.971 107.188) (end 150.1463 107.188) (width 0.25) (layer F.Cu) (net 9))
 (segment (start 160.147 102.806) (end 157.9748 104.9782) (width 0.25) (layer F.Cu) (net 9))
 (segment (start 157.9748 104.9782) (end 152.3561 104.9782) (width 0.25) (layer F.Cu) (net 9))
 (segment (start 152.3561 104.9782) (end 150.1463 107.188) (width 0.25) (layer F.Cu) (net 9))
 (segment (start 162.051 94.17) (end 160.464 92.583) (width 0.25) (layer F.Cu) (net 15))
 (segment (start 161.7672 99.8982) (end 162.051 99.6144) (width 0.25) (layer F.Cu) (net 15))
 (segment (start 162.051 99.6144) (end 162.051 94.17) (width 0.25) (layer F.Cu) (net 15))
 (segment (start 162.051 94.17) (end 162.1988 94.17) (width 0.25) (layer F.Cu) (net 15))
 (segment (start 162.1988 94.17) (end 162.9874 93.3814) (width 0.25) (layer F.Cu) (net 15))
 (segment (start 162.9874 93.3814) (end 162.9874 87.0779) (width 0.25) (layer F.Cu) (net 15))
 (segment (start 162.9874 87.0779) (end 162.2696 86.3601) (width 0.25) (layer F.Cu) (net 15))
 (segment (start 162.2696 86.3601) (end 161.2575 86.3601) (width 0.25) (layer F.Cu) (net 15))
 (segment (start 161.2575 86.3601) (end 160.4757 85.5783) (width 0.25) (layer F.Cu) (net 15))
 (segment (start 160.4757 85.5783) (end 160.4757 83.8083) (width 0.25) (layer F.Cu) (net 15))
 (segment (start 160.4757 83.8083) (end 161.734 82.55) (width 0.25) (layer F.Cu) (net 15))
 (segment (start 147.2634 112.5272) (end 152.4144 117.6782) (width 0.25) (layer F.Cu) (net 15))
 (segment (start 152.4144 117.6782) (end 153.9837 117.6782) (width 0.25) (layer F.Cu) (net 15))
 (segment (start 153.9837 117.6782) (end 157.7374 121.4319) (width 0.25) (layer F.Cu) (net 15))
 (segment (start 157.7374 121.4319) (end 157.7374 122.5952) (width 0.25) (layer F.Cu) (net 15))
 (segment (start 157.7374 122.5952) (end 160.2333 125.0911) (width 0.25) (layer F.Cu) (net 15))
 (segment (start 160.2333 125.0911) (end 161.5631 125.0911) (width 0.25) (layer F.Cu) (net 15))
 (segment (start 161.5631 125.0911) (end 164.0313 122.6229) (width 0.25) (layer F.Cu) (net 15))
 (segment (start 164.0313 122.6229) (end 164.0313 79.2119) (width 0.25) (layer F.Cu) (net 15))
 (segment (start 164.0313 79.2119) (end 160.5876 75.7682) (width 0.25) (layer F.Cu) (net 15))
 (segment (start 160.5876 75.7682) (end 153.226 75.7682) (width 0.25) (layer F.Cu) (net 15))
 (segment (start 161.7672 99.8982) (end 150.3744 99.8982) (width 0.25) (layer F.Cu) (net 15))
 (segment (start 150.3744 99.8982) (end 147.2634 103.0092) (width 0.25) (layer F.Cu) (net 15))
 (segment (start 147.2634 103.0092) (end 147.2634 112.5272) (width 0.25) (layer F.Cu) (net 15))
 (segment (start 147.2634 112.5272) (end 142.0813 117.7093) (width 0.25) (layer F.Cu) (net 15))
 (segment (start 142.0813 117.7093) (end 137.986 117.7093) (width 0.25) (layer F.Cu) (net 15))
 (segment (start 137.986 121.4882) (end 137.986 118.9482) (width 0.25) (layer F.Cu) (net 15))
 (segment (start 137.986 122.1076) (end 137.986 121.4882) (width 0.25) (layer F.Cu) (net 15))
 (segment (start 137.986 122.1076) (end 137.986 122.7271) (width 0.25) (layer F.Cu) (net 15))
 (segment (start 137.986 122.7271) (end 136.6801 124.033) (width 0.25) (layer F.Cu) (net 15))
 (segment (start 136.6801 124.033) (end 130.7448 124.033) (width 0.25) (layer F.Cu) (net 15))
 (segment (start 130.7448 124.033) (end 129.566 122.8542) (width 0.25) (layer F.Cu) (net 15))
 (segment (start 129.566 122.8542) (end 129.566 86.0292) (width 0.25) (layer F.Cu) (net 15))
 (segment (start 129.566 86.0292) (end 133.477 82.1182) (width 0.25) (layer F.Cu) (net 15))
 (segment (start 133.477 82.1182) (end 138.7797 82.1182) (width 0.25) (layer F.Cu) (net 15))
 (segment (start 138.7797 82.1182) (end 140.5103 80.3876) (width 0.25) (layer F.Cu) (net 15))
 (segment (start 140.5103 80.3876) (end 140.5103 80.1115) (width 0.25) (layer F.Cu) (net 15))
 (segment (start 140.5103 80.1115) (end 141.4086 79.2132) (width 0.25) (layer F.Cu) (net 15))
 (segment (start 141.4086 79.2132) (end 143.0764 79.2132) (width 0.25) (layer F.Cu) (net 15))
 (segment (start 143.0764 79.2132) (end 143.0764 73.0141) (width 0.25) (layer F.Cu) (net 15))
 (segment (start 143.0764 73.0141) (end 143.383 72.7075) (width 0.25) (layer F.Cu) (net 15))
 (segment (start 143.3713 87.63) (end 143.3713 79.5081) (width 0.25) (layer F.Cu) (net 15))
 (segment (start 143.3713 79.5081) (end 143.0764 79.2132) (width 0.25) (layer F.Cu) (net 15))
 (segment (start 160.338 109.5187) (end 161.2942 109.5187) (width 0.25) (layer F.Cu) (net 15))
 (segment (start 161.2942 109.5187) (end 161.7672 109.0457) (width 0.25) (layer F.Cu) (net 15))
 (segment (start 161.7672 109.0457) (end 161.7672 99.8982) (width 0.25) (layer F.Cu) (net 15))
 (segment (start 137.986 118.9482) (end 137.986 117.7093) (width 0.25) (layer F.Cu) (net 15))
 (segment (start 160.338 110.744) (end 160.338 109.5187) (width 0.25) (layer F.Cu) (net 15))
 (segment (start 141.796 87.63) (end 143.3713 87.63) (width 0.25) (layer F.Cu) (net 15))
 (segment (start 131.699 99.314) (end 134.9248 96.0882) (width 0.25) (layer F.Cu) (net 10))
 (segment (start 134.9248 96.0882) (end 137.986 96.0882) (width 0.25) (layer F.Cu) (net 10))
 (segment (start 137.986 101.1682) (end 137.986 102.4071) (width 0.25) (layer F.Cu) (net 12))
 (segment (start 131.826 110.808) (end 131.826 107.7923) (width 0.25) (layer F.Cu) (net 12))
 (segment (start 131.826 107.7923) (end 137.2112 102.4071) (width 0.25) (layer F.Cu) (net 12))
 (segment (start 137.2112 102.4071) (end 137.986 102.4071) (width 0.25) (layer F.Cu) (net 12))
 (segment (start 137.986 107.4871) (end 137.2112 107.4871) (width 0.25) (layer F.Cu) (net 14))
 (segment (start 137.2112 107.4871) (end 134.0239 110.6744) (width 0.25) (layer F.Cu) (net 14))
 (segment (start 134.0239 110.6744) (end 134.0239 119.7861) (width 0.25) (layer F.Cu) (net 14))
 (segment (start 134.0239 119.7861) (end 131.382 122.428) (width 0.25) (layer F.Cu) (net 14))
 (segment (start 137.986 106.2482) (end 137.986 107.4871) (width 0.25) (layer F.Cu) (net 14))
 (segment (start 137.986 98.6282) (end 137.986 99.8671) (width 0.25) (layer F.Cu) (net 11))
 (segment (start 131.826 105.156) (end 137.1149 99.8671) (width 0.25) (layer F.Cu) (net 11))
 (segment (start 137.1149 99.8671) (end 137.986 99.8671) (width 0.25) (layer F.Cu) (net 11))
 (segment (start 137.986 103.7082) (end 137.986 104.9471) (width 0.25) (layer F.Cu) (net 13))
 (segment (start 131.572 116.459) (end 133.4015 114.6295) (width 0.25) (layer F.Cu) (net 13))
 (segment (start 133.4015 114.6295) (end 133.4015 108.7568) (width 0.25) (layer F.Cu) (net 13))
 (segment (start 133.4015 108.7568) (end 137.2112 104.9471) (width 0.25) (layer F.Cu) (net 13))
 (segment (start 137.2112 104.9471) (end 137.986 104.9471) (width 0.25) (layer F.Cu) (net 13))
 (segment (start 137.986 91.0082) (end 137.986 89.7693) (width 0.25) (layer F.Cu) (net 6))
 (segment (start 137.986 89.7693) (end 138.7603 89.7693) (width 0.25) (layer F.Cu) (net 6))
 (segment (start 138.7603 89.7693) (end 140.2207 88.3089) (width 0.25) (layer F.Cu) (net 6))
 (segment (start 140.2207 88.3089) (end 140.2207 85.09) (width 0.25) (layer F.Cu) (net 6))
 (segment (start 141.796 85.09) (end 140.2207 85.09) (width 0.25) (layer F.Cu) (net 6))
 (segment (start 140.2207 85.09) (end 140.2207 82.0928) (width 0.25) (layer F.Cu) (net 6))
 (segment (start 140.2207 82.0928) (end 141.732 80.5815) (width 0.25) (layer F.Cu) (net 6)))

